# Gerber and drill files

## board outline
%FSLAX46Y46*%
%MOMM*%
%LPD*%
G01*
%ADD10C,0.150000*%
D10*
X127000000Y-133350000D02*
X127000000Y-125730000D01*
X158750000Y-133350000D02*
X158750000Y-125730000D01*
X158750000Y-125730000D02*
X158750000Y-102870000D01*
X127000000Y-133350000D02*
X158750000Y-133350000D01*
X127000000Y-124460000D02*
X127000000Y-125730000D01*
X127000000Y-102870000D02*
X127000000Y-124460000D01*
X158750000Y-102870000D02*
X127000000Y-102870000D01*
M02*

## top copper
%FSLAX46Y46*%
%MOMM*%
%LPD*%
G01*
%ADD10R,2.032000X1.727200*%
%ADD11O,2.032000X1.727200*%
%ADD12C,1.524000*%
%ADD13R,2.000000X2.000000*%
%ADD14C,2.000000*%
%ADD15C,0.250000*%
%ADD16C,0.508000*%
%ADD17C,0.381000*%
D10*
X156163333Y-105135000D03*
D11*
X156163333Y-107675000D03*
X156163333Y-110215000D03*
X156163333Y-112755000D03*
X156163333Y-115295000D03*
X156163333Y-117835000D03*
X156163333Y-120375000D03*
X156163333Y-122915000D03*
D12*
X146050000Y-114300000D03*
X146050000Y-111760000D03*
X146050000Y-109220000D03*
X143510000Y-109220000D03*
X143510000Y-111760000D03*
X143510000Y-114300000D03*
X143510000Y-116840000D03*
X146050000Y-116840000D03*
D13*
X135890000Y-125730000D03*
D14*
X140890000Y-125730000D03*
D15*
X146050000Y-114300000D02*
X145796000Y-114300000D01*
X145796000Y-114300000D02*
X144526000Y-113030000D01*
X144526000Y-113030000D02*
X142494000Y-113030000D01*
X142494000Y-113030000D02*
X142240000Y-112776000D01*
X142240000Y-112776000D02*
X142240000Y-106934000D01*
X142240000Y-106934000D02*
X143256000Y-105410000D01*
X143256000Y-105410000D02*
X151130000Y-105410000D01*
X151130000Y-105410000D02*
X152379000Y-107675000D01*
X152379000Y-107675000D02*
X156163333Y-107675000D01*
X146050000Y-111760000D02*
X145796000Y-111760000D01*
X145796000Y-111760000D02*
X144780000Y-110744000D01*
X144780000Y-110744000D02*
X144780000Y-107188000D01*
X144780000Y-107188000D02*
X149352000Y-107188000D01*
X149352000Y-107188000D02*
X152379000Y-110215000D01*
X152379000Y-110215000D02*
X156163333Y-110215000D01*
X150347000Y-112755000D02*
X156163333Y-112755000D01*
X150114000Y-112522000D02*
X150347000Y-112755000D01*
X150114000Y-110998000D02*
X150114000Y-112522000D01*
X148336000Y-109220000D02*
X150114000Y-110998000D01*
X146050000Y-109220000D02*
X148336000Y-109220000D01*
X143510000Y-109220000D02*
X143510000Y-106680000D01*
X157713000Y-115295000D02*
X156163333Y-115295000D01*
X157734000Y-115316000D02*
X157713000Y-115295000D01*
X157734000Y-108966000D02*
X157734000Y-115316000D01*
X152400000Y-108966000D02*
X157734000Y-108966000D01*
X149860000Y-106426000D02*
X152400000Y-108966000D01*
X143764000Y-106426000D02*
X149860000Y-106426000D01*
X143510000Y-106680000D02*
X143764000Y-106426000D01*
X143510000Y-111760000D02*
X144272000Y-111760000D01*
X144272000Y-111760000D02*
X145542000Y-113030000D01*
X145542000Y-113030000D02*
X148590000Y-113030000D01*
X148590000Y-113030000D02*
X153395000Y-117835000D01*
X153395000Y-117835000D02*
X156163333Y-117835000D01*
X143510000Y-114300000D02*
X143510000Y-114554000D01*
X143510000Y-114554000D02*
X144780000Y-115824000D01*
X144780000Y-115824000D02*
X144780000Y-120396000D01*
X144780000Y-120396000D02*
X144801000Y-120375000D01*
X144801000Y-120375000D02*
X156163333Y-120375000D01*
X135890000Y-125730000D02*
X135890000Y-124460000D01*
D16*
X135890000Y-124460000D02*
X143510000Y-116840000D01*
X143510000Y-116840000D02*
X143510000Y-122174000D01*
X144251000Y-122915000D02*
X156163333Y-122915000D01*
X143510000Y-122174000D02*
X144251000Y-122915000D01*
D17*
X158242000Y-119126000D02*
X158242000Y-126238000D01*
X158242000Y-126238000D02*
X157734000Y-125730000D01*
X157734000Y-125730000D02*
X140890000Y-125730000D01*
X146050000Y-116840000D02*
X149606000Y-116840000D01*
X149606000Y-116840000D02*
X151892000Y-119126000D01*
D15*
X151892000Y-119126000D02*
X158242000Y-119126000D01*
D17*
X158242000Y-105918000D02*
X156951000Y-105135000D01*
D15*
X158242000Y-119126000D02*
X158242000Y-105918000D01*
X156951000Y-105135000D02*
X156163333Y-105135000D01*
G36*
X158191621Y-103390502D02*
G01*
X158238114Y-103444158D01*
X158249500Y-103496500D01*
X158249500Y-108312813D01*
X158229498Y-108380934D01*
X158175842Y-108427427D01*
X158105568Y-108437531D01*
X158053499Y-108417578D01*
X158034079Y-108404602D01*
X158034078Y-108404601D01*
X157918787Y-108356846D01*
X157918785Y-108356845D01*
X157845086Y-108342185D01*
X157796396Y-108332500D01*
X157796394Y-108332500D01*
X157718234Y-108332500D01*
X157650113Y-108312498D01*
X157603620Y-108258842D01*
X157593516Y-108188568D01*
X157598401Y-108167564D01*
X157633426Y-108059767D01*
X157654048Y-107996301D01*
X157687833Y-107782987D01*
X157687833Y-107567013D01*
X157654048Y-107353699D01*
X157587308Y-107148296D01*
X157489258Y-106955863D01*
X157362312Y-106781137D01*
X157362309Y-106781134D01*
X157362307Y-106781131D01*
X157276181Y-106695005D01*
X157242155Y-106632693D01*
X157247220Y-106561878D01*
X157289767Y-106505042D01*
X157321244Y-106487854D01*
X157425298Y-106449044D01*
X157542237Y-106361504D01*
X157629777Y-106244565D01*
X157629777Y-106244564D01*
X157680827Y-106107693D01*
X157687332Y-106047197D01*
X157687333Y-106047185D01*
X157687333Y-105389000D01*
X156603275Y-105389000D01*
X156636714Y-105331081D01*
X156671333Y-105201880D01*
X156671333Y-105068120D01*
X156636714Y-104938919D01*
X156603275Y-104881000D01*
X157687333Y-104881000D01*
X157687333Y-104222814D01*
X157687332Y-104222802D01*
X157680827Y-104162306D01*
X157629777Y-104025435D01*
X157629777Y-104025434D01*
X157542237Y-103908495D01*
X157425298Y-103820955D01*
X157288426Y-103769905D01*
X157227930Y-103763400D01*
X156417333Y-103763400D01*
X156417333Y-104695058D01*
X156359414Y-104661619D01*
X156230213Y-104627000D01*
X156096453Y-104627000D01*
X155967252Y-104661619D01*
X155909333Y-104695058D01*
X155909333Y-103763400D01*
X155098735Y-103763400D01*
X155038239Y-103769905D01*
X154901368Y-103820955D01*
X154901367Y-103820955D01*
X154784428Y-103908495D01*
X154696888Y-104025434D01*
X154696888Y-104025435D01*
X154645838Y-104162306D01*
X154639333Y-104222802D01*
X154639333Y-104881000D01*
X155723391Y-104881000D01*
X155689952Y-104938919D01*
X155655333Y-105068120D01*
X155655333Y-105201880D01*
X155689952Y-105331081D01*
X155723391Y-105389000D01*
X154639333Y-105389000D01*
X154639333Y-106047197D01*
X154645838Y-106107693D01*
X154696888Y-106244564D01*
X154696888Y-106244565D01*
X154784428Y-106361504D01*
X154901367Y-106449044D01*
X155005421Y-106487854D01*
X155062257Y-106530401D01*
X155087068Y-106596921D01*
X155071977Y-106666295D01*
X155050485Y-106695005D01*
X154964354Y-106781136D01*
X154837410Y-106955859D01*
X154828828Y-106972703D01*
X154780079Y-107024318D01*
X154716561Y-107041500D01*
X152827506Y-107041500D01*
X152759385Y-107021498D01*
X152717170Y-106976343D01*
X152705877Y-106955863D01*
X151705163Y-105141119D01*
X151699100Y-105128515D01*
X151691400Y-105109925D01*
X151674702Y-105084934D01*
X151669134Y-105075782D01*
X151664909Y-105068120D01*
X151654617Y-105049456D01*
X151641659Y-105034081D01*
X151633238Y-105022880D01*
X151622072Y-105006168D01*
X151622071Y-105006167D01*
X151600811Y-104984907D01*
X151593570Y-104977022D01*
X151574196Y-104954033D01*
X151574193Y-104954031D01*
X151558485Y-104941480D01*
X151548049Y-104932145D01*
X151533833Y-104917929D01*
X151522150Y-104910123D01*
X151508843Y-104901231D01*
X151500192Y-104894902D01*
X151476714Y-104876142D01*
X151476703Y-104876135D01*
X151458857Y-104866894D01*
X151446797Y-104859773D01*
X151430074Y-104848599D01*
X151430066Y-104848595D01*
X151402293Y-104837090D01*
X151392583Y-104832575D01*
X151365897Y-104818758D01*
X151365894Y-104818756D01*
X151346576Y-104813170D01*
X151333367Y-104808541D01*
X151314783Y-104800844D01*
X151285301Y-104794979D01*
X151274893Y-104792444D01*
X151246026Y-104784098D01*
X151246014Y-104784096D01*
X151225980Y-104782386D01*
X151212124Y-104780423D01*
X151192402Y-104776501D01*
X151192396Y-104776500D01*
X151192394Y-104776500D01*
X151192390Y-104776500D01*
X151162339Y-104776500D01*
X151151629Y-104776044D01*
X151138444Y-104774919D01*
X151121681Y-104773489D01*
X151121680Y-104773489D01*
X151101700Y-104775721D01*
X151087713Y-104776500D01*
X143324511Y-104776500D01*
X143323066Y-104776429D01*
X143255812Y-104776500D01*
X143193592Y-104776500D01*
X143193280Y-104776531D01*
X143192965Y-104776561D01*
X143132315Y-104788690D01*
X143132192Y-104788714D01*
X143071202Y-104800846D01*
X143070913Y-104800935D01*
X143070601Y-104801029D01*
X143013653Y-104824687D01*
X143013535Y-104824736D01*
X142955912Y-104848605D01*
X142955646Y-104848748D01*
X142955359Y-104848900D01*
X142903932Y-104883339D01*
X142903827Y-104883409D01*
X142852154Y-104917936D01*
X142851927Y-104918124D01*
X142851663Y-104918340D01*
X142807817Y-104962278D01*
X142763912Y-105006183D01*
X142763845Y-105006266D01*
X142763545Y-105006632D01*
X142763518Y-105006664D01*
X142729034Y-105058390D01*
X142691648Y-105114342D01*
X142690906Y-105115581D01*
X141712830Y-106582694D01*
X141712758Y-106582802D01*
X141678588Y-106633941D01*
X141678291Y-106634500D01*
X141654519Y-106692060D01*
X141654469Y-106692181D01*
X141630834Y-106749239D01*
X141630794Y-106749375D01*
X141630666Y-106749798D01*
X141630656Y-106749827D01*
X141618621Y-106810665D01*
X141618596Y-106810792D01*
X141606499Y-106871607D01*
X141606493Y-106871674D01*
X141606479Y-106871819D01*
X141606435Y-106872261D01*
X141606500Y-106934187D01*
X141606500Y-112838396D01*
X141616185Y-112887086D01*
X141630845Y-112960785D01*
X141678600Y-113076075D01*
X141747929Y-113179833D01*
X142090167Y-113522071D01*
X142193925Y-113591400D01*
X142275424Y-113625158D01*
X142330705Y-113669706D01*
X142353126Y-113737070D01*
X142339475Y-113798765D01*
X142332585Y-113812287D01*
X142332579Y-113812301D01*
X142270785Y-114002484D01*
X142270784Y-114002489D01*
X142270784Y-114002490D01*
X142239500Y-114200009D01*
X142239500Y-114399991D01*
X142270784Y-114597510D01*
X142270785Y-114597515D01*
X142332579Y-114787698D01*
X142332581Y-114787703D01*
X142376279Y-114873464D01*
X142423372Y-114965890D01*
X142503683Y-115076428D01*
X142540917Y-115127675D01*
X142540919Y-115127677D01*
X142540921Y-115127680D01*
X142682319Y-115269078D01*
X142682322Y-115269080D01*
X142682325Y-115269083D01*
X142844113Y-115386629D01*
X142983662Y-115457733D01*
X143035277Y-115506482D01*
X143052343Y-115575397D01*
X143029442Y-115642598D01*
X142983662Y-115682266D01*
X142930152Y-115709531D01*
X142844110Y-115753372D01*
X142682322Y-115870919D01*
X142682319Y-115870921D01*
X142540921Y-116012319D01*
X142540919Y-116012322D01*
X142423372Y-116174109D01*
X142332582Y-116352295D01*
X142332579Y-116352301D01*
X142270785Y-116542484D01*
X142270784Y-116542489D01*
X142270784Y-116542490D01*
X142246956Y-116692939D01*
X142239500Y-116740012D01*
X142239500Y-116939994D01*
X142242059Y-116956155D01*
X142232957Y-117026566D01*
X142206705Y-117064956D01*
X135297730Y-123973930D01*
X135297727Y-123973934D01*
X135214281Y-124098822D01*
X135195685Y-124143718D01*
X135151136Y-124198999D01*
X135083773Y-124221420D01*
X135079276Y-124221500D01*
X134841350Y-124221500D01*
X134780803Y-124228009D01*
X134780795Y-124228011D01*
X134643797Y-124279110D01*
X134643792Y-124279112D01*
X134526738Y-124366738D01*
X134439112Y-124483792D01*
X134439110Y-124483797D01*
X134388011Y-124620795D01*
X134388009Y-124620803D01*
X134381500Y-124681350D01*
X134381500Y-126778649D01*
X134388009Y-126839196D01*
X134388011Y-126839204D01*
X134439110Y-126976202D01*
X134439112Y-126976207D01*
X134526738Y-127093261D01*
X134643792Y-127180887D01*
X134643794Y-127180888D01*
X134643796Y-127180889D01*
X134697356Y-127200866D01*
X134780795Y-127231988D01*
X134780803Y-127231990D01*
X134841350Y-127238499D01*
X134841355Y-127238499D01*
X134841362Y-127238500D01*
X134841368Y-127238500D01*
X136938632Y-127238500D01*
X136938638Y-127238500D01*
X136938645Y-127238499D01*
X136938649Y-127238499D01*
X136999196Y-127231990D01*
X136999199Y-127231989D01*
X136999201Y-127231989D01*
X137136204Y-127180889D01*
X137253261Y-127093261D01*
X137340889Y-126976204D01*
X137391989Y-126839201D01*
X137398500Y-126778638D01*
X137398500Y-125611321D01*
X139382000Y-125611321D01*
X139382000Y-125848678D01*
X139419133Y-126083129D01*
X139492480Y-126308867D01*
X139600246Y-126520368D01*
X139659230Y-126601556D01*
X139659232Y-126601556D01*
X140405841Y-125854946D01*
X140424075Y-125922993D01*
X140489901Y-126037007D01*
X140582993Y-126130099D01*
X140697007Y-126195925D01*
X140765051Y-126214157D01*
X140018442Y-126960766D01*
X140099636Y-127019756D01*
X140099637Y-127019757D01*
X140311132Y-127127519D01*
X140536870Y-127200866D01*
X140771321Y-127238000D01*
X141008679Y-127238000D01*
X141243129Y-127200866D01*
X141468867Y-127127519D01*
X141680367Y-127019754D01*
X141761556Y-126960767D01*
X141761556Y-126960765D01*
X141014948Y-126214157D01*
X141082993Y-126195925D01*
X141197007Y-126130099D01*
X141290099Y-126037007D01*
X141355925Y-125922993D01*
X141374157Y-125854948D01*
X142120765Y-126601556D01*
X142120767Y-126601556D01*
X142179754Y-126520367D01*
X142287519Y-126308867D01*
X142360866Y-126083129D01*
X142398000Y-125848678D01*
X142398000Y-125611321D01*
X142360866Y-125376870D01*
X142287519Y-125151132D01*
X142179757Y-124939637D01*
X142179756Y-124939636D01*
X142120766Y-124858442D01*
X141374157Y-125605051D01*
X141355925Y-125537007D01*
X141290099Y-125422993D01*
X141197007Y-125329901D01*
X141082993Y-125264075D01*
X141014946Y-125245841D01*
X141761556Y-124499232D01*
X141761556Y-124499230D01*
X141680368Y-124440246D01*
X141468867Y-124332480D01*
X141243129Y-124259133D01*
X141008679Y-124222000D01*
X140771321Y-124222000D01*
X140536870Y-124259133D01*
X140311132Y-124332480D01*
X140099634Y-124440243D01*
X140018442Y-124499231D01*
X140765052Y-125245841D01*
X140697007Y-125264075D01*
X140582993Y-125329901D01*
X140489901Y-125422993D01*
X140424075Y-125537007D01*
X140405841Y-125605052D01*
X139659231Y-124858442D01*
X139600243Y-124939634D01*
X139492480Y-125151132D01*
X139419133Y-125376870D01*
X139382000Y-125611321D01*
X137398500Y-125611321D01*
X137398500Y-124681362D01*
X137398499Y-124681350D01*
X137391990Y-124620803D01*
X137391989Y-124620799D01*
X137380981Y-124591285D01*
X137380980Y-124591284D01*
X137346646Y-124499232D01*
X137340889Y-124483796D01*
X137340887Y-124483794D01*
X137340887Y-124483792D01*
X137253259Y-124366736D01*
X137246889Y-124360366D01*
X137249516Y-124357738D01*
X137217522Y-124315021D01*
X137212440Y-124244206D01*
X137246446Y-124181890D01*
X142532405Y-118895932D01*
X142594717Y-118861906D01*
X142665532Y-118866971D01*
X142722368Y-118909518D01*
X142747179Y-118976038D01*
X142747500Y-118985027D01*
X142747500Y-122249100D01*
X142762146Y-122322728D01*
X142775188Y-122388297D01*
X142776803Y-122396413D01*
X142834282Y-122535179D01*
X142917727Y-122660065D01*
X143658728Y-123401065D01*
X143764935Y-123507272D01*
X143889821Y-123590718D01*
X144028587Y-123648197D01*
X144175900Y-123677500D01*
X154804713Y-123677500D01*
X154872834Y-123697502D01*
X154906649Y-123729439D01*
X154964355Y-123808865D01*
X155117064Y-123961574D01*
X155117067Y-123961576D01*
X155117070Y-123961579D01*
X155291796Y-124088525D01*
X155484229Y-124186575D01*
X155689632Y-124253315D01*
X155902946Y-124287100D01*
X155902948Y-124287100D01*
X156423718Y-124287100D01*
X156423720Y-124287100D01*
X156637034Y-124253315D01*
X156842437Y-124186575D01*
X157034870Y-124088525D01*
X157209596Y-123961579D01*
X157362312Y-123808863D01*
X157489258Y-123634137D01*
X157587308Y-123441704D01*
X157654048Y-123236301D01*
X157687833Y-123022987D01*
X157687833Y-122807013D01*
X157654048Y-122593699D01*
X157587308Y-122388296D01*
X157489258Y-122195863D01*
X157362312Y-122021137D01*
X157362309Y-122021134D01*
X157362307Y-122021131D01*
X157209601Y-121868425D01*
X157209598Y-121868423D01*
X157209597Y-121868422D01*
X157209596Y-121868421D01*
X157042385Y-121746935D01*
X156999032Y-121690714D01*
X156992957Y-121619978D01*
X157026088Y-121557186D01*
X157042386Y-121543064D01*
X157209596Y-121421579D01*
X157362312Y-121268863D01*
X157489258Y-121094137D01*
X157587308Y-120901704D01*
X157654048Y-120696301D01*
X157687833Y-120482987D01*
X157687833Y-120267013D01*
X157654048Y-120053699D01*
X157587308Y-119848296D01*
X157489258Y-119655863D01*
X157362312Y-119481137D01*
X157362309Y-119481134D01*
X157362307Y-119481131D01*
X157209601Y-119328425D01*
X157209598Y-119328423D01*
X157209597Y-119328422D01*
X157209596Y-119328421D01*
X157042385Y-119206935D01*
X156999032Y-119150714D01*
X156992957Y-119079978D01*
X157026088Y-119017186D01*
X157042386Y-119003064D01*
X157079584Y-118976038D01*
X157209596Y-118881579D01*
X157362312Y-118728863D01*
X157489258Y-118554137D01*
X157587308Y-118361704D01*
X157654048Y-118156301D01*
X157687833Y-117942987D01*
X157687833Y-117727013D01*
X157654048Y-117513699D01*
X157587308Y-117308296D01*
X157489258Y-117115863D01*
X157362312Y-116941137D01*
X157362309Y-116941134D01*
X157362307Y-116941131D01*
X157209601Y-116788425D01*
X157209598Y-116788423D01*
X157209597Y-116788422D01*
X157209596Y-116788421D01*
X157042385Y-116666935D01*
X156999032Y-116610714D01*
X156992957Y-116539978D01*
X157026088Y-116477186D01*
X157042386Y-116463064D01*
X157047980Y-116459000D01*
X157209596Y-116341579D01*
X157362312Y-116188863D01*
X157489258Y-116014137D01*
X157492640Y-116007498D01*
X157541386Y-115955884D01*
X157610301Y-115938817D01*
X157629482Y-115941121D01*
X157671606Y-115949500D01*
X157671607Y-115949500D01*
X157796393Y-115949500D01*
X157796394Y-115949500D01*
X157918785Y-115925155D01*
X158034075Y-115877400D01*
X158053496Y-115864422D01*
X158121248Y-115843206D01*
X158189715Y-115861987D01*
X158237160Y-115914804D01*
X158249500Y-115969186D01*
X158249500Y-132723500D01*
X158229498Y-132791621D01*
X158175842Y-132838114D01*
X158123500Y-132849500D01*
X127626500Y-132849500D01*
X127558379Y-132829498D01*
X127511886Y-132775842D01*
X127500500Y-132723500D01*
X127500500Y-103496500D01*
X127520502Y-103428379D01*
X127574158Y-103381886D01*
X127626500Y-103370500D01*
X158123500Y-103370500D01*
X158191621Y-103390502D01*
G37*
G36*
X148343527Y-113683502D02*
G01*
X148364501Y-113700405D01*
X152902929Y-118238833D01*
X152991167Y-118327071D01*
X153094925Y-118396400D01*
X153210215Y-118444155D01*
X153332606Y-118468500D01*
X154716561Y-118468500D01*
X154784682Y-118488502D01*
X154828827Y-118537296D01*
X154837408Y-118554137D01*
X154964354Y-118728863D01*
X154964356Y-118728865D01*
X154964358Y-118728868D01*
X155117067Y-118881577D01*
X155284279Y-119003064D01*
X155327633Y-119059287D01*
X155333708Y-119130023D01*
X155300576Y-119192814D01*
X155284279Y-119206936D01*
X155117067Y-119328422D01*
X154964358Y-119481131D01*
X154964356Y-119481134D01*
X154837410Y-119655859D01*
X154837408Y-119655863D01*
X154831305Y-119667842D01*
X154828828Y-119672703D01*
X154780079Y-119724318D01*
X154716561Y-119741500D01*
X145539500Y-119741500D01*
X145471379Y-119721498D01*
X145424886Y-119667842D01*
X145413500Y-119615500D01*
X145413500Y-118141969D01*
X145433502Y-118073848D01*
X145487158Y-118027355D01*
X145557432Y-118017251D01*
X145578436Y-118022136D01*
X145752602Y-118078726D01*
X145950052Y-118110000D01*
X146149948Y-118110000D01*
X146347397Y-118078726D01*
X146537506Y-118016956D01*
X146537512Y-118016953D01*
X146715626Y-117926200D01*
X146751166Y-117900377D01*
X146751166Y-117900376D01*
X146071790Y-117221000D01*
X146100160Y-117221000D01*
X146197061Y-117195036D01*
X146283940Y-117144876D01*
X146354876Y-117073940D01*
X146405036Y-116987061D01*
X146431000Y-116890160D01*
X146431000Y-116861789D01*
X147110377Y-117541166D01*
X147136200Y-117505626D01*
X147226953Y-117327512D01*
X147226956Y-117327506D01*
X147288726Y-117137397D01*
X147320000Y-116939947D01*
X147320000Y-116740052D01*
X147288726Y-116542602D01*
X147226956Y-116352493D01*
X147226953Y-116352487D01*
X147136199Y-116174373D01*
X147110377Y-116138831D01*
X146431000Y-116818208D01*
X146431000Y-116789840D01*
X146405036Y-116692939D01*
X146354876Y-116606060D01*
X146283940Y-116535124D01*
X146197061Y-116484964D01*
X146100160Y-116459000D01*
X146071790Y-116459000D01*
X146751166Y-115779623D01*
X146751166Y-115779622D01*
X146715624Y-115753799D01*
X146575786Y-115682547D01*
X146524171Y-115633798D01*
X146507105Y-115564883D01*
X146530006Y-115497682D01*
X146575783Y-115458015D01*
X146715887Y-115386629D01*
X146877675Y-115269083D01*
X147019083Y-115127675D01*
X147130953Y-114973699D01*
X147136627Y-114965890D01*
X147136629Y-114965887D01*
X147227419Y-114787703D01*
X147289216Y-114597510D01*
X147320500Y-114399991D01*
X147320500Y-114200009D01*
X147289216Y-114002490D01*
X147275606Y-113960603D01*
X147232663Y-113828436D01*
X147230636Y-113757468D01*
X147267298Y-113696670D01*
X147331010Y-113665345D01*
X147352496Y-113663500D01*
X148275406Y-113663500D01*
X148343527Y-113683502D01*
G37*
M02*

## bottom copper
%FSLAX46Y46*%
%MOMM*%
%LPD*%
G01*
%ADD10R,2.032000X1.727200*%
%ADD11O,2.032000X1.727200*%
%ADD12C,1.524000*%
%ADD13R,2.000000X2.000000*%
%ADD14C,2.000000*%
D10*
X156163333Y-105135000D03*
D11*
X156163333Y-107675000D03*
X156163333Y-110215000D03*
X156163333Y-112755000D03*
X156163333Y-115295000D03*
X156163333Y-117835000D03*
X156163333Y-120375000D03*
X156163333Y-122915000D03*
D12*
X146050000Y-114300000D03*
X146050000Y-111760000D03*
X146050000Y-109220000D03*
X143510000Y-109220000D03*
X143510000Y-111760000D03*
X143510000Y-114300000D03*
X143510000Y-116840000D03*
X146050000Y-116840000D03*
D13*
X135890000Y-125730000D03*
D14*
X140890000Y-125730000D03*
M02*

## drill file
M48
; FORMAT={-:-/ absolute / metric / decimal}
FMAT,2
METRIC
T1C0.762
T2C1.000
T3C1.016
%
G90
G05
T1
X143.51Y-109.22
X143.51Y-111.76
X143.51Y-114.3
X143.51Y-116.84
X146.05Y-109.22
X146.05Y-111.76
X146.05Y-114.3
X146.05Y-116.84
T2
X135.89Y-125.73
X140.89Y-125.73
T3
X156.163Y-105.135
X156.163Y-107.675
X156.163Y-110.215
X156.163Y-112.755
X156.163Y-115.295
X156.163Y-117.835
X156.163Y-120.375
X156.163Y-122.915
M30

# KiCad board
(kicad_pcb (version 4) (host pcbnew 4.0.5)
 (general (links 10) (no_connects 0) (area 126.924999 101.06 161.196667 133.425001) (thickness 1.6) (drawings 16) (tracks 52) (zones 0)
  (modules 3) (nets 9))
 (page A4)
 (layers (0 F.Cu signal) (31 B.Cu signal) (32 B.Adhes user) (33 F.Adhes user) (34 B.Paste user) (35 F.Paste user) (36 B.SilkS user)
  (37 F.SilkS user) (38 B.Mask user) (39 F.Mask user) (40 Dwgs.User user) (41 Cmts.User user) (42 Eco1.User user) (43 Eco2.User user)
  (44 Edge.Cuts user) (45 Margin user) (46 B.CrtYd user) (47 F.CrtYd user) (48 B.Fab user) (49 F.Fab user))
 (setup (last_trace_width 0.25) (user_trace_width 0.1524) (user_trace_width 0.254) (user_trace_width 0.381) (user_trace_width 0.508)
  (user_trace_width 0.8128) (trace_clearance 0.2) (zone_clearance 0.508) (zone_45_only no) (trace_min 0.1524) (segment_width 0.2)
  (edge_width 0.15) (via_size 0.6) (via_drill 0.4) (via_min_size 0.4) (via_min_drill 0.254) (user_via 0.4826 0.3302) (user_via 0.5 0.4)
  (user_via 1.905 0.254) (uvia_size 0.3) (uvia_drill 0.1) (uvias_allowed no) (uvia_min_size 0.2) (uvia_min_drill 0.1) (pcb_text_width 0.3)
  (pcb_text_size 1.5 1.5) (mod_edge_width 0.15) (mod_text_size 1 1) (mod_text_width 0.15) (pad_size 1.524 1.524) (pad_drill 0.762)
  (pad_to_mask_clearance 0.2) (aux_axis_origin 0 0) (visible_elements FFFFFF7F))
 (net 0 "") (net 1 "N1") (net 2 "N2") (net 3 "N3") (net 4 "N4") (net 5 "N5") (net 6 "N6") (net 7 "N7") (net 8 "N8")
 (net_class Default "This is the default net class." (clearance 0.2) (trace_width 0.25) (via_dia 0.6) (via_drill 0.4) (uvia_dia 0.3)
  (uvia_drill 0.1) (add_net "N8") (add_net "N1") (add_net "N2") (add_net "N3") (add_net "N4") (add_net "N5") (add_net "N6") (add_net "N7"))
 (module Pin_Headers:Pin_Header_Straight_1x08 (layer F.Cu) (at 156.163333 105.135)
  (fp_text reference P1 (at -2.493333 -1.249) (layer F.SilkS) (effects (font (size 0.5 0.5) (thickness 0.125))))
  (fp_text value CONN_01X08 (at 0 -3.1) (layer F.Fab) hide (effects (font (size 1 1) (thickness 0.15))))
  (pad 1 thru_hole rect (at 0 0) (size 2.032 1.7272) (drill 1.016) (layers *.Cu *.Mask) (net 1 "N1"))
  (pad 2 thru_hole oval (at 0 2.54) (size 2.032 1.7272) (drill 1.016) (layers *.Cu *.Mask) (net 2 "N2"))
  (pad 3 thru_hole oval (at 0 5.08) (size 2.032 1.7272) (drill 1.016) (layers *.Cu *.Mask) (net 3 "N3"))
  (pad 4 thru_hole oval (at 0 7.62) (size 2.032 1.7272) (drill 1.016) (layers *.Cu *.Mask) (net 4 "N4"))
  (pad 5 thru_hole oval (at 0 10.16) (size 2.032 1.7272) (drill 1.016) (layers *.Cu *.Mask) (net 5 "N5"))
  (pad 6 thru_hole oval (at 0 12.7) (size 2.032 1.7272) (drill 1.016) (layers *.Cu *.Mask) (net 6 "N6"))
  (pad 7 thru_hole oval (at 0 15.24) (size 2.032 1.7272) (drill 1.016) (layers *.Cu *.Mask) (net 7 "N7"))
  (pad 8 thru_hole oval (at 0 17.78) (size 2.032 1.7272) (drill 1.016) (layers *.Cu *.Mask) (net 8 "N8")))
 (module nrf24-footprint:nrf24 (layer F.Cu) (at 135.89 114.3)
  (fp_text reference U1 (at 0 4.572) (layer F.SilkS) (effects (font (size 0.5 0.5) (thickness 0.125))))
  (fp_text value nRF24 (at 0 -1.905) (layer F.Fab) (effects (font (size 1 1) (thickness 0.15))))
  (pad 1 thru_hole circle (at 10.16 0) (size 1.524 1.524) (drill 0.762) (layers *.Cu *.Mask) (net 2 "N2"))
  (pad 2 thru_hole circle (at 10.16 -2.54) (size 1.524 1.524) (drill 0.762) (layers *.Cu *.Mask) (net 3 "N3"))
  (pad 3 thru_hole circle (at 10.16 -5.08) (size 1.524 1.524) (drill 0.762) (layers *.Cu *.Mask) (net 4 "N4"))
  (pad 4 thru_hole circle (at 7.62 -5.08) (size 1.524 1.524) (drill 0.762) (layers *.Cu *.Mask) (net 5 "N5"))
  (pad 5 thru_hole circle (at 7.62 -2.54) (size 1.524 1.524) (drill 0.762) (layers *.Cu *.Mask) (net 6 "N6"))
  (pad 6 thru_hole circle (at 7.62 0) (size 1.524 1.524) (drill 0.762) (layers *.Cu *.Mask) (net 7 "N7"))
  (pad 7 thru_hole circle (at 7.62 2.54) (size 1.524 1.524) (drill 0.762) (layers *.Cu *.Mask) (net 8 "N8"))
  (pad 0 thru_hole circle (at 10.16 2.54) (size 1.524 1.524) (drill 0.762) (layers *.Cu *.Mask) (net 1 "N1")))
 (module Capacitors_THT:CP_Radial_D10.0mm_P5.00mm (layer F.Cu) (at 135.89 125.73)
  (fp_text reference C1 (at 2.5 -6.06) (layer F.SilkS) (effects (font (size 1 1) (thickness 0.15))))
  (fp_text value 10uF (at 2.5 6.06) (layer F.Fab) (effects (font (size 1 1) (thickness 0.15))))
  (pad 1 thru_hole rect (at 0 0) (size 2 2) (drill 1) (layers *.Cu *.Mask) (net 8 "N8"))
  (pad 2 thru_hole circle (at 5 0) (size 2 2) (drill 1) (layers *.Cu *.Mask) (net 1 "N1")))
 (gr_line (start 127 133.35) (end 127 125.73) (angle 90) (layer Edge.Cuts) (width 0.15))
 (gr_line (start 158.75 133.35) (end 158.75 125.73) (angle 90) (layer Edge.Cuts) (width 0.15))
 (gr_line (start 158.75 125.73) (end 158.75 102.87) (angle 90) (layer Edge.Cuts) (width 0.15))
 (gr_line (start 127 133.35) (end 158.75 133.35) (angle 90) (layer Edge.Cuts) (width 0.15))
 (gr_line (start 127 124.46) (end 127 125.73) (angle 90) (layer Edge.Cuts) (width 0.15))
 (gr_line (start 127 102.87) (end 127 124.46) (angle 90) (layer Edge.Cuts) (width 0.15))
 (gr_line (start 158.75 102.87) (end 127 102.87) (angle 90) (layer Edge.Cuts) (width 0.15))
 (segment (start 146.05 114.3) (end 145.796 114.3) (width 0.25) (layer F.Cu) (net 2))
 (segment (start 145.796 114.3) (end 144.526 113.03) (width 0.25) (layer F.Cu) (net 2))
 (segment (start 144.526 113.03) (end 142.494 113.03) (width 0.25) (layer F.Cu) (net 2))
 (segment (start 142.494 113.03) (end 142.24 112.776) (width 0.25) (layer F.Cu) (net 2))
 (segment (start 142.24 112.776) (end 142.24 106.934) (width 0.25) (layer F.Cu) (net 2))
 (segment (start 142.24 106.934) (end 143.256 105.41) (width 0.25) (layer F.Cu) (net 2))
 (segment (start 143.256 105.41) (end 151.13 105.41) (width 0.25) (layer F.Cu) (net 2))
 (segment (start 151.13 105.41) (end 152.379 107.675) (width 0.25) (layer F.Cu) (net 2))
 (segment (start 152.379 107.675) (end 156.163333 107.675) (width 0.25) (layer F.Cu) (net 2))
 (segment (start 146.05 111.76) (end 145.796 111.76) (width 0.25) (layer F.Cu) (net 3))
 (segment (start 145.796 111.76) (end 144.78 110.744) (width 0.25) (layer F.Cu) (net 3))
 (segment (start 144.78 110.744) (end 144.78 107.188) (width 0.25) (layer F.Cu) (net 3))
 (segment (start 144.78 107.188) (end 149.352 107.188) (width 0.25) (layer F.Cu) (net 3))
 (segment (start 149.352 107.188) (end 152.379 110.215) (width 0.25) (layer F.Cu) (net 3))
 (segment (start 152.379 110.215) (end 156.163333 110.215) (width 0.25) (layer F.Cu) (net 3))
 (segment (start 150.347 112.755) (end 156.163333 112.755) (width 0.25) (layer F.Cu) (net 4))
 (segment (start 150.114 112.522) (end 150.347 112.755) (width 0.25) (layer F.Cu) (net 4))
 (segment (start 150.114 110.998) (end 150.114 112.522) (width 0.25) (layer F.Cu) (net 4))
 (segment (start 148.336 109.22) (end 150.114 110.998) (width 0.25) (layer F.Cu) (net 4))
 (segment (start 146.05 109.22) (end 148.336 109.22) (width 0.25) (layer F.Cu) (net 4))
 (segment (start 143.51 109.22) (end 143.51 106.68) (width 0.25) (layer F.Cu) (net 5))
 (segment (start 157.713 115.295) (end 156.163333 115.295) (width 0.25) (layer F.Cu) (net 5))
 (segment (start 157.734 115.316) (end 157.713 115.295) (width 0.25) (layer F.Cu) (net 5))
 (segment (start 157.734 108.966) (end 157.734 115.316) (width 0.25) (layer F.Cu) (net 5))
 (segment (start 152.4 108.966) (end 157.734 108.966) (width 0.25) (layer F.Cu) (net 5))
 (segment (start 149.86 106.426) (end 152.4 108.966) (width 0.25) (layer F.Cu) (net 5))
 (segment (start 143.764 106.426) (end 149.86 106.426) (width 0.25) (layer F.Cu) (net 5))
 (segment (start 143.51 106.68) (end 143.764 106.426) (width 0.25) (layer F.Cu) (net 5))
 (segment (start 143.51 111.76) (end 144.272 111.76) (width 0.25) (layer F.Cu) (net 6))
 (segment (start 144.272 111.76) (end 145.542 113.03) (width 0.25) (layer F.Cu) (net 6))
 (segment (start 145.542 113.03) (end 148.59 113.03) (width 0.25) (layer F.Cu) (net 6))
 (segment (start 148.59 113.03) (end 153.395 117.835) (width 0.25) (layer F.Cu) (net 6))
 (segment (start 153.395 117.835) (end 156.163333 117.835) (width 0.25) (layer F.Cu) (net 6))
 (segment (start 143.51 114.3) (end 143.51 114.554) (width 0.25) (layer F.Cu) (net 7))
 (segment (start 143.51 114.554) (end 144.78 115.824) (width 0.25) (layer F.Cu) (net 7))
 (segment (start 144.78 115.824) (end 144.78 120.396) (width 0.25) (layer F.Cu) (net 7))
 (segment (start 144.78 120.396) (end 144.801 120.375) (width 0.25) (layer F.Cu) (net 7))
 (segment (start 144.801 120.375) (end 156.163333 120.375) (width 0.25) (layer F.Cu) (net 7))
 (segment (start 135.89 125.73) (end 135.89 124.46) (width 0.25) (layer F.Cu) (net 8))
 (segment (start 135.89 124.46) (end 143.51 116.84) (width 0.508) (layer F.Cu) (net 8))
 (segment (start 143.51 116.84) (end 143.51 122.174) (width 0.508) (layer F.Cu) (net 8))
 (segment (start 144.251 122.915) (end 156.163333 122.915) (width 0.508) (layer F.Cu) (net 8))
 (segment (start 143.51 122.174) (end 144.251 122.915) (width 0.508) (layer F.Cu) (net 8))
 (segment (start 158.242 119.126) (end 158.242 126.238) (width 0.381) (layer F.Cu) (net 1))
 (segment (start 158.242 126.238) (end 157.734 125.73) (width 0.381) (layer F.Cu) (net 1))
 (segment (start 157.734 125.73) (end 140.89 125.73) (width 0.381) (layer F.Cu) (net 1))
 (segment (start 146.05 116.84) (end 149.606 116.84) (width 0.381) (layer F.Cu) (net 1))
 (segment (start 149.606 116.84) (end 151.892 119.126) (width 0.381) (layer F.Cu) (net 1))
 (segment (start 151.892 119.126) (end 158.242 119.126) (width 0.25) (layer F.Cu) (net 1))
 (segment (start 158.242 105.918) (end 156.951 105.135) (width 0.381) (layer F.Cu) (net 1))
 (segment (start 158.242 119.126) (end 158.242 105.918) (width 0.25) (layer F.Cu) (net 1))
 (segment (start 156.951 105.135) (end 156.163333 105.135) (width 0.25) (layer F.Cu) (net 1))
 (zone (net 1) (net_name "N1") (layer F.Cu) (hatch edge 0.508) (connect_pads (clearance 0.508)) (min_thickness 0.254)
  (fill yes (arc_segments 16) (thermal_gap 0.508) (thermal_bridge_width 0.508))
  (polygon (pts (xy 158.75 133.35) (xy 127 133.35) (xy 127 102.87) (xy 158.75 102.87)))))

